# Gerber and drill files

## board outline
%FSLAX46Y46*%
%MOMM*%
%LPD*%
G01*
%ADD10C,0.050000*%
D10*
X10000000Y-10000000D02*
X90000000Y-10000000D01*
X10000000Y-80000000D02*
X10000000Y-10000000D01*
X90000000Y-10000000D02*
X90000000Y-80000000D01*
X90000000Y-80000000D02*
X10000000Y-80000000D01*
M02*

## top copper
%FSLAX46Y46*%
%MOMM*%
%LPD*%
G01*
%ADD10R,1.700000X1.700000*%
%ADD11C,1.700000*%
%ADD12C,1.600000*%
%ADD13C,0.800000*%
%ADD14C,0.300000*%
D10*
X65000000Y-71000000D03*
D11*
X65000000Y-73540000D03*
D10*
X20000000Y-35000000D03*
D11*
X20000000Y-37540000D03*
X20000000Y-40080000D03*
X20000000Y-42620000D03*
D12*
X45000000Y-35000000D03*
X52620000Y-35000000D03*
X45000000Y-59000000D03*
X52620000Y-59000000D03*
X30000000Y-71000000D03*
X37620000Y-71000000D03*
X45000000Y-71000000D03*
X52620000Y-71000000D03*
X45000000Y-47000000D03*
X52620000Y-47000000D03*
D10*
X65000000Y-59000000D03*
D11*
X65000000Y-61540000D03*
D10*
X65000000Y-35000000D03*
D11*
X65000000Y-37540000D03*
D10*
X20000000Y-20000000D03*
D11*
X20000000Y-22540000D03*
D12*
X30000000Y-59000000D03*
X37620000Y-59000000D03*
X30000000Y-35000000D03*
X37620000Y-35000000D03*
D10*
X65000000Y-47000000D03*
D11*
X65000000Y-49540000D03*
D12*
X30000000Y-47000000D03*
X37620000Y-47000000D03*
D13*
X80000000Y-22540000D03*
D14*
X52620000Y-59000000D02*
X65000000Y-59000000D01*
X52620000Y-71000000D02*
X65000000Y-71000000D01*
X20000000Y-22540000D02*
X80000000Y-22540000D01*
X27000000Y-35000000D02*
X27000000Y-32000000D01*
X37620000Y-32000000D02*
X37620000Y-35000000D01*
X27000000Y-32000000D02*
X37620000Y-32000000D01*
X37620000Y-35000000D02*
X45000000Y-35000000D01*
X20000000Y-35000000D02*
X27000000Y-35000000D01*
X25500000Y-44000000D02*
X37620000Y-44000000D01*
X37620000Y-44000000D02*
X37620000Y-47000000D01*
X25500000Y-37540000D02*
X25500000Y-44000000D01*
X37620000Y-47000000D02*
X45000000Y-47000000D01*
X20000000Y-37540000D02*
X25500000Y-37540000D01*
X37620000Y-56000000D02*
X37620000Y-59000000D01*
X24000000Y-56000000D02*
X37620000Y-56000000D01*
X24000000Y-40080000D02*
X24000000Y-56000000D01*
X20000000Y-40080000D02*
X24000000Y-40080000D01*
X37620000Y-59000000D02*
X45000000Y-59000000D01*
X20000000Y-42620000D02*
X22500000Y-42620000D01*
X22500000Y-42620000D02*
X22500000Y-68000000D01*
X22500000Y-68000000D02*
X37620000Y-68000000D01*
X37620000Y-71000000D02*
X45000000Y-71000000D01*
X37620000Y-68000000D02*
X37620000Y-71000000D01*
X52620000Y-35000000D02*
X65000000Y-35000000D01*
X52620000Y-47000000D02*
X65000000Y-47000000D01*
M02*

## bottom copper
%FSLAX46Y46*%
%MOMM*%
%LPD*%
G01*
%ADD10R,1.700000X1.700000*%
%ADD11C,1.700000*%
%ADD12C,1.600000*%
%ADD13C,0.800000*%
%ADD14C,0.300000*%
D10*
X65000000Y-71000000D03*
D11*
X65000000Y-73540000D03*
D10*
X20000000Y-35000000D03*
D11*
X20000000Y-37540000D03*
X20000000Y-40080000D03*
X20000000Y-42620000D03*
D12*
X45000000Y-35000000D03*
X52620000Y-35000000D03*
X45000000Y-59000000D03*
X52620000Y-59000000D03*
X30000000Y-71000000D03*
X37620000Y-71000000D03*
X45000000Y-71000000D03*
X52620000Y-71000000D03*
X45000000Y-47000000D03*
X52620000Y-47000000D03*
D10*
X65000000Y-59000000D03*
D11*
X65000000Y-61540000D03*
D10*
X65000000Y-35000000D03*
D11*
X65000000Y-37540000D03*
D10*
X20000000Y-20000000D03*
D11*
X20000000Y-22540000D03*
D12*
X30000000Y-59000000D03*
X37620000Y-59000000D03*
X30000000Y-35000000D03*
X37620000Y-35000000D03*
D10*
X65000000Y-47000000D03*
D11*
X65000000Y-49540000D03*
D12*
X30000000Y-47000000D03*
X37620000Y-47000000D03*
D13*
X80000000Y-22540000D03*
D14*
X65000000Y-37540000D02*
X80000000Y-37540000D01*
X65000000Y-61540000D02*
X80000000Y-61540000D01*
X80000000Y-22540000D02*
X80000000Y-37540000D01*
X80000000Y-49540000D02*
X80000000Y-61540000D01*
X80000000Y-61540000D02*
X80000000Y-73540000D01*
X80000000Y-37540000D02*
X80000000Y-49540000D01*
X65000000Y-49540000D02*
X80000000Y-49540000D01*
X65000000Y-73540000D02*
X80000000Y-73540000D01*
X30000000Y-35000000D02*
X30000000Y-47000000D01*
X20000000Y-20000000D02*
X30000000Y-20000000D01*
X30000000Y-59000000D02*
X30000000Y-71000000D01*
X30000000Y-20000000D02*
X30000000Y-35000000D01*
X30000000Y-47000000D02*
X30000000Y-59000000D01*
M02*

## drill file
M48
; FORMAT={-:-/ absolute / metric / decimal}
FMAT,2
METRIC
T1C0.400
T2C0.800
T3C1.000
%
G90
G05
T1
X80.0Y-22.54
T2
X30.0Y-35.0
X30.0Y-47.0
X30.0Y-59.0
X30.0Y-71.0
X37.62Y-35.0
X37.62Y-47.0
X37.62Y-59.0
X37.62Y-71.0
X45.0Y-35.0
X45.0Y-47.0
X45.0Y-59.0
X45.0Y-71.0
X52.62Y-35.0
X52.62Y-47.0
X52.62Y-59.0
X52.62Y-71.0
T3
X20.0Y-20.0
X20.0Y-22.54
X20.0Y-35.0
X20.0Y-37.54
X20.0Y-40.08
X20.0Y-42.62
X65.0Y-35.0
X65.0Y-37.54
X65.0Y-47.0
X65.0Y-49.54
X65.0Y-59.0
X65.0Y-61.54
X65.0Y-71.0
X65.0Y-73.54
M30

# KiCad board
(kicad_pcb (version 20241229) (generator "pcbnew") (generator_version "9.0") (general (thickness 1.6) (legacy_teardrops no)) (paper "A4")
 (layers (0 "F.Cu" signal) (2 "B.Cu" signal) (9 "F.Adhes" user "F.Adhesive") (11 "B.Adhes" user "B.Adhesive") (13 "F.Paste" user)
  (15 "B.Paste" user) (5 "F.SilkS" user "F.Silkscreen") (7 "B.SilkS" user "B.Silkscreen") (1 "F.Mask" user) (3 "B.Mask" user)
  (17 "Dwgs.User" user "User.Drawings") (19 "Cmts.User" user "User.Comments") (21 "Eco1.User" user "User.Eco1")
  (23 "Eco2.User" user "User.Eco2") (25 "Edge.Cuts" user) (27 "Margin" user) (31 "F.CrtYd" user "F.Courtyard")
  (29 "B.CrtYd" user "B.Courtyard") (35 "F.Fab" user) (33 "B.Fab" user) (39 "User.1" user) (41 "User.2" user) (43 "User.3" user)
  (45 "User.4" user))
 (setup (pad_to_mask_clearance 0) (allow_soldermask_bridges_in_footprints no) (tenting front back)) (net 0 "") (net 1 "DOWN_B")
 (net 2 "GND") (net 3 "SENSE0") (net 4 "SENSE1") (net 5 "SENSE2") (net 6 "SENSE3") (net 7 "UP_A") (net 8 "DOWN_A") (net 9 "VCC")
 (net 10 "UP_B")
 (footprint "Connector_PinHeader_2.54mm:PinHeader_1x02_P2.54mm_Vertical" (layer "F.Cu") (at 65 71)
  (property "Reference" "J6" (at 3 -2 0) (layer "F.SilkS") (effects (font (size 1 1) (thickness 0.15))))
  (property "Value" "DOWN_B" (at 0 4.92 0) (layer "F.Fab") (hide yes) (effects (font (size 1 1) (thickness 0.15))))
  (pad "1" thru_hole rect (at 0 0) (size 1.7 1.7) (drill 1) (layers "*.Cu" "*.Mask") (remove_unused_layers no) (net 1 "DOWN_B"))
  (pad "2" thru_hole circle (at 0 2.54) (size 1.7 1.7) (drill 1) (layers "*.Cu" "*.Mask") (remove_unused_layers no) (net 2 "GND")))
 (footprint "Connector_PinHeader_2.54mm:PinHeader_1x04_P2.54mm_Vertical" (layer "F.Cu") (at 20 35)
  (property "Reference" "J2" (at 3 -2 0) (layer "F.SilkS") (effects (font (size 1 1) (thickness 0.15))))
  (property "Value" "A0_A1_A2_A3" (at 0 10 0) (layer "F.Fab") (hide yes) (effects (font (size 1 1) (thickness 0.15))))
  (pad "1" thru_hole rect (at 0 0) (size 1.7 1.7) (drill 1) (layers "*.Cu" "*.Mask") (remove_unused_layers no) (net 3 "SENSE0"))
  (pad "2" thru_hole circle (at 0 2.54) (size 1.7 1.7) (drill 1) (layers "*.Cu" "*.Mask") (remove_unused_layers no) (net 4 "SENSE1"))
  (pad "3" thru_hole circle (at 0 5.08) (size 1.7 1.7) (drill 1) (layers "*.Cu" "*.Mask") (remove_unused_layers no) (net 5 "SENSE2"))
  (pad "4" thru_hole circle (at 0 7.62) (size 1.7 1.7) (drill 1) (layers "*.Cu" "*.Mask") (remove_unused_layers no) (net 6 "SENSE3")))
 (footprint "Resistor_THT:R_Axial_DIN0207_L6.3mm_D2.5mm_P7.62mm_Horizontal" (layer "F.Cu") (at 45 35)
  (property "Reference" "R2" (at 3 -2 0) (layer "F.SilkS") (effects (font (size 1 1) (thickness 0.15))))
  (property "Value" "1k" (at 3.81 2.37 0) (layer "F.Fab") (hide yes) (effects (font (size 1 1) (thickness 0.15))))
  (pad "1" thru_hole circle (at 0 0) (size 1.6 1.6) (drill 0.8) (layers "*.Cu" "*.Mask") (remove_unused_layers no) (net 3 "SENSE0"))
  (pad "2" thru_hole circle (at 7.62 0) (size 1.6 1.6) (drill 0.8) (layers "*.Cu" "*.Mask") (remove_unused_layers no) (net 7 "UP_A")))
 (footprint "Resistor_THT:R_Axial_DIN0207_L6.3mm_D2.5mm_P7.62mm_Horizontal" (layer "F.Cu") (at 45 59)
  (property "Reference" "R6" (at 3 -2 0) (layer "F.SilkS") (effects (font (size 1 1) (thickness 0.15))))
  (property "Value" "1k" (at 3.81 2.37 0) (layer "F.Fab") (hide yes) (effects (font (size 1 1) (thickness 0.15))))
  (pad "1" thru_hole circle (at 0 0) (size 1.6 1.6) (drill 0.8) (layers "*.Cu" "*.Mask") (remove_unused_layers no) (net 5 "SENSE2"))
  (pad "2" thru_hole circle (at 7.62 0) (size 1.6 1.6) (drill 0.8) (layers "*.Cu" "*.Mask") (remove_unused_layers no) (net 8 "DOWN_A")))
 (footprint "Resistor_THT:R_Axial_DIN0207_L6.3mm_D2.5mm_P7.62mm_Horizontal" (layer "F.Cu") (at 30 71)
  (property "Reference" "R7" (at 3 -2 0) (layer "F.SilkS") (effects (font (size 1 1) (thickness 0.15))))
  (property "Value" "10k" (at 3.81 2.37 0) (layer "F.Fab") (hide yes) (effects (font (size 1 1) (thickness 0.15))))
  (pad "1" thru_hole circle (at 0 0) (size 1.6 1.6) (drill 0.8) (layers "*.Cu" "*.Mask") (remove_unused_layers no) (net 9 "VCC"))
  (pad "2" thru_hole circle (at 7.62 0) (size 1.6 1.6) (drill 0.8) (layers "*.Cu" "*.Mask") (remove_unused_layers no) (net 6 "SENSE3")))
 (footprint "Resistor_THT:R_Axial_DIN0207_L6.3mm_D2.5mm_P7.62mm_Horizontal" (layer "F.Cu") (at 45 71)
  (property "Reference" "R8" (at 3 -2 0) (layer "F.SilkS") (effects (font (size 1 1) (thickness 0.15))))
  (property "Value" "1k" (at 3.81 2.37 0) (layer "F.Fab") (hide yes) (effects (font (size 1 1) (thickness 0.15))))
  (pad "1" thru_hole circle (at 0 0) (size 1.6 1.6) (drill 0.8) (layers "*.Cu" "*.Mask") (remove_unused_layers no) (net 6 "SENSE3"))
  (pad "2" thru_hole circle (at 7.62 0) (size 1.6 1.6) (drill 0.8) (layers "*.Cu" "*.Mask") (remove_unused_layers no) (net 1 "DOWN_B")))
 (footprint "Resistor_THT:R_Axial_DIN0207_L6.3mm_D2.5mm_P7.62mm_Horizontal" (layer "F.Cu") (at 45 47)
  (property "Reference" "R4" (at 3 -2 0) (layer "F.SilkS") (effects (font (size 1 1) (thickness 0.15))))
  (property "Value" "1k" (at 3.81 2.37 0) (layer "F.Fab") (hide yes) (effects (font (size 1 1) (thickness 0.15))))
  (pad "1" thru_hole circle (at 0 0) (size 1.6 1.6) (drill 0.8) (layers "*.Cu" "*.Mask") (remove_unused_layers no) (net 4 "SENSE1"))
  (pad "2" thru_hole circle (at 7.62 0) (size 1.6 1.6) (drill 0.8) (layers "*.Cu" "*.Mask") (remove_unused_layers no) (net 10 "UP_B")))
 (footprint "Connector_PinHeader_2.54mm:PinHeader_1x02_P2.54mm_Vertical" (layer "F.Cu") (at 65 59)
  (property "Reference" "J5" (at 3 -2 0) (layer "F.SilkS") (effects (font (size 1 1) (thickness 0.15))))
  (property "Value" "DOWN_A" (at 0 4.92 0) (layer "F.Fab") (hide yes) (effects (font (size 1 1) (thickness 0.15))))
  (pad "1" thru_hole rect (at 0 0) (size 1.7 1.7) (drill 1) (layers "*.Cu" "*.Mask") (remove_unused_layers no) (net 8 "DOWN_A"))
  (pad "2" thru_hole circle (at 0 2.54) (size 1.7 1.7) (drill 1) (layers "*.Cu" "*.Mask") (remove_unused_layers no) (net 2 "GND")))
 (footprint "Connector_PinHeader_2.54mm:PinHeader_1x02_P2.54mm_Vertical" (layer "F.Cu") (at 65 35)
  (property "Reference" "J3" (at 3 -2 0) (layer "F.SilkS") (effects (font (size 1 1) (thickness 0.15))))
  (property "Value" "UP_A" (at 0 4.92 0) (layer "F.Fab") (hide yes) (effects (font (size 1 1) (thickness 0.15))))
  (pad "1" thru_hole rect (at 0 0) (size 1.7 1.7) (drill 1) (layers "*.Cu" "*.Mask") (remove_unused_layers no) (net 7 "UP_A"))
  (pad "2" thru_hole circle (at 0 2.54) (size 1.7 1.7) (drill 1) (layers "*.Cu" "*.Mask") (remove_unused_layers no) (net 2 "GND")))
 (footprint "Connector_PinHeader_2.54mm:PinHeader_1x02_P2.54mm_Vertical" (layer "F.Cu") (at 20 20)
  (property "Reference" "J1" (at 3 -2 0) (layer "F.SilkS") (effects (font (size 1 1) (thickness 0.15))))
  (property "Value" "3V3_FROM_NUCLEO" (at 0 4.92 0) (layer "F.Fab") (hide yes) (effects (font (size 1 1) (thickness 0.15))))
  (pad "1" thru_hole rect (at 0 0) (size 1.7 1.7) (drill 1) (layers "*.Cu" "*.Mask") (remove_unused_layers no) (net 9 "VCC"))
  (pad "2" thru_hole circle (at 0 2.54) (size 1.7 1.7) (drill 1) (layers "*.Cu" "*.Mask") (remove_unused_layers no) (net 2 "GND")))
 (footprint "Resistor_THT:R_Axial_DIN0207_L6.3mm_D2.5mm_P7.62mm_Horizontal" (layer "F.Cu") (at 30 59)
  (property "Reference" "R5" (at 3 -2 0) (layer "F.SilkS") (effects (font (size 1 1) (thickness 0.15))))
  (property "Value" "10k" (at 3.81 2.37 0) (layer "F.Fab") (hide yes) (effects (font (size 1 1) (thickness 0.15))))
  (pad "1" thru_hole circle (at 0 0) (size 1.6 1.6) (drill 0.8) (layers "*.Cu" "*.Mask") (remove_unused_layers no) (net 9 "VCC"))
  (pad "2" thru_hole circle (at 7.62 0) (size 1.6 1.6) (drill 0.8) (layers "*.Cu" "*.Mask") (remove_unused_layers no) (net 5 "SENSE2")))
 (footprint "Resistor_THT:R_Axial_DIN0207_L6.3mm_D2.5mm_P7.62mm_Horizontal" (layer "F.Cu") (at 30 35)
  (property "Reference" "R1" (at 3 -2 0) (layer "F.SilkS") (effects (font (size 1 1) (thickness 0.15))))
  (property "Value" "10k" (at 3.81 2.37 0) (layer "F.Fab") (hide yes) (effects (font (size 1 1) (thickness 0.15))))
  (pad "1" thru_hole circle (at 0 0) (size 1.6 1.6) (drill 0.8) (layers "*.Cu" "*.Mask") (remove_unused_layers no) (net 9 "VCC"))
  (pad "2" thru_hole circle (at 7.62 0) (size 1.6 1.6) (drill 0.8) (layers "*.Cu" "*.Mask") (remove_unused_layers no) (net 3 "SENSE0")))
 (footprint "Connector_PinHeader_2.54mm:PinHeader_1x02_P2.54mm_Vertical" (layer "F.Cu") (at 65 47)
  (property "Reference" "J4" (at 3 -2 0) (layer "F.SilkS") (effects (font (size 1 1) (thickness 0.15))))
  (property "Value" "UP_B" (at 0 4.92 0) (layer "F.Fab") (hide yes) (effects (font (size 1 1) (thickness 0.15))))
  (pad "1" thru_hole rect (at 0 0) (size 1.7 1.7) (drill 1) (layers "*.Cu" "*.Mask") (remove_unused_layers no) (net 10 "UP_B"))
  (pad "2" thru_hole circle (at 0 2.54) (size 1.7 1.7) (drill 1) (layers "*.Cu" "*.Mask") (remove_unused_layers no) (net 2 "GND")))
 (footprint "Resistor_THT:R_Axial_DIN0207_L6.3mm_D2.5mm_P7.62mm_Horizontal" (layer "F.Cu") (at 30 47)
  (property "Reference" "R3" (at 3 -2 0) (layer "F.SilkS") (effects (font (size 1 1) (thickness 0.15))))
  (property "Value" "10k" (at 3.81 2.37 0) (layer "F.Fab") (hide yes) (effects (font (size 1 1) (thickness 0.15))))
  (pad "1" thru_hole circle (at 0 0) (size 1.6 1.6) (drill 0.8) (layers "*.Cu" "*.Mask") (remove_unused_layers no) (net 9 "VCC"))
  (pad "2" thru_hole circle (at 7.62 0) (size 1.6 1.6) (drill 0.8) (layers "*.Cu" "*.Mask") (remove_unused_layers no) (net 4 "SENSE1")))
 (gr_line (start 10 10) (end 90 10) (stroke (width 0.05) (type default)) (layer "Edge.Cuts"))
 (gr_line (start 10 80) (end 10 10) (stroke (width 0.05) (type default)) (layer "Edge.Cuts"))
 (gr_line (start 90 10) (end 90 80) (stroke (width 0.05) (type default)) (layer "Edge.Cuts"))
 (gr_line (start 90 80) (end 10 80) (stroke (width 0.05) (type default)) (layer "Edge.Cuts"))
 (segment (start 52.62 59) (end 65 59) (width 0.3) (layer "F.Cu") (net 8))
 (segment (start 52.62 71) (end 65 71) (width 0.3) (layer "F.Cu") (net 1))
 (segment (start 20 22.54) (end 80 22.54) (width 0.3) (layer "F.Cu") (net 2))
 (via (at 80 22.54) (size 0.8) (drill 0.4) (layers "F.Cu" "B.Cu") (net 2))
 (segment (start 65 37.54) (end 80 37.54) (width 0.3) (layer "B.Cu") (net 2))
 (segment (start 65 61.54) (end 80 61.54) (width 0.3) (layer "B.Cu") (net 2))
 (segment (start 80 22.54) (end 80 37.54) (width 0.3) (layer "B.Cu") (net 2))
 (segment (start 80 49.54) (end 80 61.54) (width 0.3) (layer "B.Cu") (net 2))
 (segment (start 80 61.54) (end 80 73.54) (width 0.3) (layer "B.Cu") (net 2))
 (segment (start 80 37.54) (end 80 49.54) (width 0.3) (layer "B.Cu") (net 2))
 (segment (start 65 49.54) (end 80 49.54) (width 0.3) (layer "B.Cu") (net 2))
 (segment (start 65 73.54) (end 80 73.54) (width 0.3) (layer "B.Cu") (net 2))
 (segment (start 27 35) (end 27 32) (width 0.3) (layer "F.Cu") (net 3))
 (segment (start 37.62 32) (end 37.62 35) (width 0.3) (layer "F.Cu") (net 3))
 (segment (start 27 32) (end 37.62 32) (width 0.3) (layer "F.Cu") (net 3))
 (segment (start 37.62 35) (end 45 35) (width 0.3) (layer "F.Cu") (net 3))
 (segment (start 20 35) (end 27 35) (width 0.3) (layer "F.Cu") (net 3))
 (segment (start 25.5 44) (end 37.62 44) (width 0.3) (layer "F.Cu") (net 4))
 (segment (start 37.62 44) (end 37.62 47) (width 0.3) (layer "F.Cu") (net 4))
 (segment (start 25.5 37.54) (end 25.5 44) (width 0.3) (layer "F.Cu") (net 4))
 (segment (start 37.62 47) (end 45 47) (width 0.3) (layer "F.Cu") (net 4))
 (segment (start 20 37.54) (end 25.5 37.54) (width 0.3) (layer "F.Cu") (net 4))
 (segment (start 37.62 56) (end 37.62 59) (width 0.3) (layer "F.Cu") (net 5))
 (segment (start 24 56) (end 37.62 56) (width 0.3) (layer "F.Cu") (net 5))
 (segment (start 24 40.08) (end 24 56) (width 0.3) (layer "F.Cu") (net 5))
 (segment (start 20 40.08) (end 24 40.08) (width 0.3) (layer "F.Cu") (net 5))
 (segment (start 37.62 59) (end 45 59) (width 0.3) (layer "F.Cu") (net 5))
 (segment (start 20 42.62) (end 22.5 42.62) (width 0.3) (layer "F.Cu") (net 6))
 (segment (start 22.5 42.62) (end 22.5 68) (width 0.3) (layer "F.Cu") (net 6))
 (segment (start 22.5 68) (end 37.62 68) (width 0.3) (layer "F.Cu") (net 6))
 (segment (start 37.62 71) (end 45 71) (width 0.3) (layer "F.Cu") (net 6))
 (segment (start 37.62 68) (end 37.62 71) (width 0.3) (layer "F.Cu") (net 6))
 (segment (start 52.62 35) (end 65 35) (width 0.3) (layer "F.Cu") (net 7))
 (segment (start 52.62 47) (end 65 47) (width 0.3) (layer "F.Cu") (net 10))
 (segment (start 30 35) (end 30 47) (width 0.3) (layer "B.Cu") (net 9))
 (segment (start 20 20) (end 30 20) (width 0.3) (layer "B.Cu") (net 9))
 (segment (start 30 59) (end 30 71) (width 0.3) (layer "B.Cu") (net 9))
 (segment (start 30 20) (end 30 35) (width 0.3) (layer "B.Cu") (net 9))
 (segment (start 30 47) (end 30 59) (width 0.3) (layer "B.Cu") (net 9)))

